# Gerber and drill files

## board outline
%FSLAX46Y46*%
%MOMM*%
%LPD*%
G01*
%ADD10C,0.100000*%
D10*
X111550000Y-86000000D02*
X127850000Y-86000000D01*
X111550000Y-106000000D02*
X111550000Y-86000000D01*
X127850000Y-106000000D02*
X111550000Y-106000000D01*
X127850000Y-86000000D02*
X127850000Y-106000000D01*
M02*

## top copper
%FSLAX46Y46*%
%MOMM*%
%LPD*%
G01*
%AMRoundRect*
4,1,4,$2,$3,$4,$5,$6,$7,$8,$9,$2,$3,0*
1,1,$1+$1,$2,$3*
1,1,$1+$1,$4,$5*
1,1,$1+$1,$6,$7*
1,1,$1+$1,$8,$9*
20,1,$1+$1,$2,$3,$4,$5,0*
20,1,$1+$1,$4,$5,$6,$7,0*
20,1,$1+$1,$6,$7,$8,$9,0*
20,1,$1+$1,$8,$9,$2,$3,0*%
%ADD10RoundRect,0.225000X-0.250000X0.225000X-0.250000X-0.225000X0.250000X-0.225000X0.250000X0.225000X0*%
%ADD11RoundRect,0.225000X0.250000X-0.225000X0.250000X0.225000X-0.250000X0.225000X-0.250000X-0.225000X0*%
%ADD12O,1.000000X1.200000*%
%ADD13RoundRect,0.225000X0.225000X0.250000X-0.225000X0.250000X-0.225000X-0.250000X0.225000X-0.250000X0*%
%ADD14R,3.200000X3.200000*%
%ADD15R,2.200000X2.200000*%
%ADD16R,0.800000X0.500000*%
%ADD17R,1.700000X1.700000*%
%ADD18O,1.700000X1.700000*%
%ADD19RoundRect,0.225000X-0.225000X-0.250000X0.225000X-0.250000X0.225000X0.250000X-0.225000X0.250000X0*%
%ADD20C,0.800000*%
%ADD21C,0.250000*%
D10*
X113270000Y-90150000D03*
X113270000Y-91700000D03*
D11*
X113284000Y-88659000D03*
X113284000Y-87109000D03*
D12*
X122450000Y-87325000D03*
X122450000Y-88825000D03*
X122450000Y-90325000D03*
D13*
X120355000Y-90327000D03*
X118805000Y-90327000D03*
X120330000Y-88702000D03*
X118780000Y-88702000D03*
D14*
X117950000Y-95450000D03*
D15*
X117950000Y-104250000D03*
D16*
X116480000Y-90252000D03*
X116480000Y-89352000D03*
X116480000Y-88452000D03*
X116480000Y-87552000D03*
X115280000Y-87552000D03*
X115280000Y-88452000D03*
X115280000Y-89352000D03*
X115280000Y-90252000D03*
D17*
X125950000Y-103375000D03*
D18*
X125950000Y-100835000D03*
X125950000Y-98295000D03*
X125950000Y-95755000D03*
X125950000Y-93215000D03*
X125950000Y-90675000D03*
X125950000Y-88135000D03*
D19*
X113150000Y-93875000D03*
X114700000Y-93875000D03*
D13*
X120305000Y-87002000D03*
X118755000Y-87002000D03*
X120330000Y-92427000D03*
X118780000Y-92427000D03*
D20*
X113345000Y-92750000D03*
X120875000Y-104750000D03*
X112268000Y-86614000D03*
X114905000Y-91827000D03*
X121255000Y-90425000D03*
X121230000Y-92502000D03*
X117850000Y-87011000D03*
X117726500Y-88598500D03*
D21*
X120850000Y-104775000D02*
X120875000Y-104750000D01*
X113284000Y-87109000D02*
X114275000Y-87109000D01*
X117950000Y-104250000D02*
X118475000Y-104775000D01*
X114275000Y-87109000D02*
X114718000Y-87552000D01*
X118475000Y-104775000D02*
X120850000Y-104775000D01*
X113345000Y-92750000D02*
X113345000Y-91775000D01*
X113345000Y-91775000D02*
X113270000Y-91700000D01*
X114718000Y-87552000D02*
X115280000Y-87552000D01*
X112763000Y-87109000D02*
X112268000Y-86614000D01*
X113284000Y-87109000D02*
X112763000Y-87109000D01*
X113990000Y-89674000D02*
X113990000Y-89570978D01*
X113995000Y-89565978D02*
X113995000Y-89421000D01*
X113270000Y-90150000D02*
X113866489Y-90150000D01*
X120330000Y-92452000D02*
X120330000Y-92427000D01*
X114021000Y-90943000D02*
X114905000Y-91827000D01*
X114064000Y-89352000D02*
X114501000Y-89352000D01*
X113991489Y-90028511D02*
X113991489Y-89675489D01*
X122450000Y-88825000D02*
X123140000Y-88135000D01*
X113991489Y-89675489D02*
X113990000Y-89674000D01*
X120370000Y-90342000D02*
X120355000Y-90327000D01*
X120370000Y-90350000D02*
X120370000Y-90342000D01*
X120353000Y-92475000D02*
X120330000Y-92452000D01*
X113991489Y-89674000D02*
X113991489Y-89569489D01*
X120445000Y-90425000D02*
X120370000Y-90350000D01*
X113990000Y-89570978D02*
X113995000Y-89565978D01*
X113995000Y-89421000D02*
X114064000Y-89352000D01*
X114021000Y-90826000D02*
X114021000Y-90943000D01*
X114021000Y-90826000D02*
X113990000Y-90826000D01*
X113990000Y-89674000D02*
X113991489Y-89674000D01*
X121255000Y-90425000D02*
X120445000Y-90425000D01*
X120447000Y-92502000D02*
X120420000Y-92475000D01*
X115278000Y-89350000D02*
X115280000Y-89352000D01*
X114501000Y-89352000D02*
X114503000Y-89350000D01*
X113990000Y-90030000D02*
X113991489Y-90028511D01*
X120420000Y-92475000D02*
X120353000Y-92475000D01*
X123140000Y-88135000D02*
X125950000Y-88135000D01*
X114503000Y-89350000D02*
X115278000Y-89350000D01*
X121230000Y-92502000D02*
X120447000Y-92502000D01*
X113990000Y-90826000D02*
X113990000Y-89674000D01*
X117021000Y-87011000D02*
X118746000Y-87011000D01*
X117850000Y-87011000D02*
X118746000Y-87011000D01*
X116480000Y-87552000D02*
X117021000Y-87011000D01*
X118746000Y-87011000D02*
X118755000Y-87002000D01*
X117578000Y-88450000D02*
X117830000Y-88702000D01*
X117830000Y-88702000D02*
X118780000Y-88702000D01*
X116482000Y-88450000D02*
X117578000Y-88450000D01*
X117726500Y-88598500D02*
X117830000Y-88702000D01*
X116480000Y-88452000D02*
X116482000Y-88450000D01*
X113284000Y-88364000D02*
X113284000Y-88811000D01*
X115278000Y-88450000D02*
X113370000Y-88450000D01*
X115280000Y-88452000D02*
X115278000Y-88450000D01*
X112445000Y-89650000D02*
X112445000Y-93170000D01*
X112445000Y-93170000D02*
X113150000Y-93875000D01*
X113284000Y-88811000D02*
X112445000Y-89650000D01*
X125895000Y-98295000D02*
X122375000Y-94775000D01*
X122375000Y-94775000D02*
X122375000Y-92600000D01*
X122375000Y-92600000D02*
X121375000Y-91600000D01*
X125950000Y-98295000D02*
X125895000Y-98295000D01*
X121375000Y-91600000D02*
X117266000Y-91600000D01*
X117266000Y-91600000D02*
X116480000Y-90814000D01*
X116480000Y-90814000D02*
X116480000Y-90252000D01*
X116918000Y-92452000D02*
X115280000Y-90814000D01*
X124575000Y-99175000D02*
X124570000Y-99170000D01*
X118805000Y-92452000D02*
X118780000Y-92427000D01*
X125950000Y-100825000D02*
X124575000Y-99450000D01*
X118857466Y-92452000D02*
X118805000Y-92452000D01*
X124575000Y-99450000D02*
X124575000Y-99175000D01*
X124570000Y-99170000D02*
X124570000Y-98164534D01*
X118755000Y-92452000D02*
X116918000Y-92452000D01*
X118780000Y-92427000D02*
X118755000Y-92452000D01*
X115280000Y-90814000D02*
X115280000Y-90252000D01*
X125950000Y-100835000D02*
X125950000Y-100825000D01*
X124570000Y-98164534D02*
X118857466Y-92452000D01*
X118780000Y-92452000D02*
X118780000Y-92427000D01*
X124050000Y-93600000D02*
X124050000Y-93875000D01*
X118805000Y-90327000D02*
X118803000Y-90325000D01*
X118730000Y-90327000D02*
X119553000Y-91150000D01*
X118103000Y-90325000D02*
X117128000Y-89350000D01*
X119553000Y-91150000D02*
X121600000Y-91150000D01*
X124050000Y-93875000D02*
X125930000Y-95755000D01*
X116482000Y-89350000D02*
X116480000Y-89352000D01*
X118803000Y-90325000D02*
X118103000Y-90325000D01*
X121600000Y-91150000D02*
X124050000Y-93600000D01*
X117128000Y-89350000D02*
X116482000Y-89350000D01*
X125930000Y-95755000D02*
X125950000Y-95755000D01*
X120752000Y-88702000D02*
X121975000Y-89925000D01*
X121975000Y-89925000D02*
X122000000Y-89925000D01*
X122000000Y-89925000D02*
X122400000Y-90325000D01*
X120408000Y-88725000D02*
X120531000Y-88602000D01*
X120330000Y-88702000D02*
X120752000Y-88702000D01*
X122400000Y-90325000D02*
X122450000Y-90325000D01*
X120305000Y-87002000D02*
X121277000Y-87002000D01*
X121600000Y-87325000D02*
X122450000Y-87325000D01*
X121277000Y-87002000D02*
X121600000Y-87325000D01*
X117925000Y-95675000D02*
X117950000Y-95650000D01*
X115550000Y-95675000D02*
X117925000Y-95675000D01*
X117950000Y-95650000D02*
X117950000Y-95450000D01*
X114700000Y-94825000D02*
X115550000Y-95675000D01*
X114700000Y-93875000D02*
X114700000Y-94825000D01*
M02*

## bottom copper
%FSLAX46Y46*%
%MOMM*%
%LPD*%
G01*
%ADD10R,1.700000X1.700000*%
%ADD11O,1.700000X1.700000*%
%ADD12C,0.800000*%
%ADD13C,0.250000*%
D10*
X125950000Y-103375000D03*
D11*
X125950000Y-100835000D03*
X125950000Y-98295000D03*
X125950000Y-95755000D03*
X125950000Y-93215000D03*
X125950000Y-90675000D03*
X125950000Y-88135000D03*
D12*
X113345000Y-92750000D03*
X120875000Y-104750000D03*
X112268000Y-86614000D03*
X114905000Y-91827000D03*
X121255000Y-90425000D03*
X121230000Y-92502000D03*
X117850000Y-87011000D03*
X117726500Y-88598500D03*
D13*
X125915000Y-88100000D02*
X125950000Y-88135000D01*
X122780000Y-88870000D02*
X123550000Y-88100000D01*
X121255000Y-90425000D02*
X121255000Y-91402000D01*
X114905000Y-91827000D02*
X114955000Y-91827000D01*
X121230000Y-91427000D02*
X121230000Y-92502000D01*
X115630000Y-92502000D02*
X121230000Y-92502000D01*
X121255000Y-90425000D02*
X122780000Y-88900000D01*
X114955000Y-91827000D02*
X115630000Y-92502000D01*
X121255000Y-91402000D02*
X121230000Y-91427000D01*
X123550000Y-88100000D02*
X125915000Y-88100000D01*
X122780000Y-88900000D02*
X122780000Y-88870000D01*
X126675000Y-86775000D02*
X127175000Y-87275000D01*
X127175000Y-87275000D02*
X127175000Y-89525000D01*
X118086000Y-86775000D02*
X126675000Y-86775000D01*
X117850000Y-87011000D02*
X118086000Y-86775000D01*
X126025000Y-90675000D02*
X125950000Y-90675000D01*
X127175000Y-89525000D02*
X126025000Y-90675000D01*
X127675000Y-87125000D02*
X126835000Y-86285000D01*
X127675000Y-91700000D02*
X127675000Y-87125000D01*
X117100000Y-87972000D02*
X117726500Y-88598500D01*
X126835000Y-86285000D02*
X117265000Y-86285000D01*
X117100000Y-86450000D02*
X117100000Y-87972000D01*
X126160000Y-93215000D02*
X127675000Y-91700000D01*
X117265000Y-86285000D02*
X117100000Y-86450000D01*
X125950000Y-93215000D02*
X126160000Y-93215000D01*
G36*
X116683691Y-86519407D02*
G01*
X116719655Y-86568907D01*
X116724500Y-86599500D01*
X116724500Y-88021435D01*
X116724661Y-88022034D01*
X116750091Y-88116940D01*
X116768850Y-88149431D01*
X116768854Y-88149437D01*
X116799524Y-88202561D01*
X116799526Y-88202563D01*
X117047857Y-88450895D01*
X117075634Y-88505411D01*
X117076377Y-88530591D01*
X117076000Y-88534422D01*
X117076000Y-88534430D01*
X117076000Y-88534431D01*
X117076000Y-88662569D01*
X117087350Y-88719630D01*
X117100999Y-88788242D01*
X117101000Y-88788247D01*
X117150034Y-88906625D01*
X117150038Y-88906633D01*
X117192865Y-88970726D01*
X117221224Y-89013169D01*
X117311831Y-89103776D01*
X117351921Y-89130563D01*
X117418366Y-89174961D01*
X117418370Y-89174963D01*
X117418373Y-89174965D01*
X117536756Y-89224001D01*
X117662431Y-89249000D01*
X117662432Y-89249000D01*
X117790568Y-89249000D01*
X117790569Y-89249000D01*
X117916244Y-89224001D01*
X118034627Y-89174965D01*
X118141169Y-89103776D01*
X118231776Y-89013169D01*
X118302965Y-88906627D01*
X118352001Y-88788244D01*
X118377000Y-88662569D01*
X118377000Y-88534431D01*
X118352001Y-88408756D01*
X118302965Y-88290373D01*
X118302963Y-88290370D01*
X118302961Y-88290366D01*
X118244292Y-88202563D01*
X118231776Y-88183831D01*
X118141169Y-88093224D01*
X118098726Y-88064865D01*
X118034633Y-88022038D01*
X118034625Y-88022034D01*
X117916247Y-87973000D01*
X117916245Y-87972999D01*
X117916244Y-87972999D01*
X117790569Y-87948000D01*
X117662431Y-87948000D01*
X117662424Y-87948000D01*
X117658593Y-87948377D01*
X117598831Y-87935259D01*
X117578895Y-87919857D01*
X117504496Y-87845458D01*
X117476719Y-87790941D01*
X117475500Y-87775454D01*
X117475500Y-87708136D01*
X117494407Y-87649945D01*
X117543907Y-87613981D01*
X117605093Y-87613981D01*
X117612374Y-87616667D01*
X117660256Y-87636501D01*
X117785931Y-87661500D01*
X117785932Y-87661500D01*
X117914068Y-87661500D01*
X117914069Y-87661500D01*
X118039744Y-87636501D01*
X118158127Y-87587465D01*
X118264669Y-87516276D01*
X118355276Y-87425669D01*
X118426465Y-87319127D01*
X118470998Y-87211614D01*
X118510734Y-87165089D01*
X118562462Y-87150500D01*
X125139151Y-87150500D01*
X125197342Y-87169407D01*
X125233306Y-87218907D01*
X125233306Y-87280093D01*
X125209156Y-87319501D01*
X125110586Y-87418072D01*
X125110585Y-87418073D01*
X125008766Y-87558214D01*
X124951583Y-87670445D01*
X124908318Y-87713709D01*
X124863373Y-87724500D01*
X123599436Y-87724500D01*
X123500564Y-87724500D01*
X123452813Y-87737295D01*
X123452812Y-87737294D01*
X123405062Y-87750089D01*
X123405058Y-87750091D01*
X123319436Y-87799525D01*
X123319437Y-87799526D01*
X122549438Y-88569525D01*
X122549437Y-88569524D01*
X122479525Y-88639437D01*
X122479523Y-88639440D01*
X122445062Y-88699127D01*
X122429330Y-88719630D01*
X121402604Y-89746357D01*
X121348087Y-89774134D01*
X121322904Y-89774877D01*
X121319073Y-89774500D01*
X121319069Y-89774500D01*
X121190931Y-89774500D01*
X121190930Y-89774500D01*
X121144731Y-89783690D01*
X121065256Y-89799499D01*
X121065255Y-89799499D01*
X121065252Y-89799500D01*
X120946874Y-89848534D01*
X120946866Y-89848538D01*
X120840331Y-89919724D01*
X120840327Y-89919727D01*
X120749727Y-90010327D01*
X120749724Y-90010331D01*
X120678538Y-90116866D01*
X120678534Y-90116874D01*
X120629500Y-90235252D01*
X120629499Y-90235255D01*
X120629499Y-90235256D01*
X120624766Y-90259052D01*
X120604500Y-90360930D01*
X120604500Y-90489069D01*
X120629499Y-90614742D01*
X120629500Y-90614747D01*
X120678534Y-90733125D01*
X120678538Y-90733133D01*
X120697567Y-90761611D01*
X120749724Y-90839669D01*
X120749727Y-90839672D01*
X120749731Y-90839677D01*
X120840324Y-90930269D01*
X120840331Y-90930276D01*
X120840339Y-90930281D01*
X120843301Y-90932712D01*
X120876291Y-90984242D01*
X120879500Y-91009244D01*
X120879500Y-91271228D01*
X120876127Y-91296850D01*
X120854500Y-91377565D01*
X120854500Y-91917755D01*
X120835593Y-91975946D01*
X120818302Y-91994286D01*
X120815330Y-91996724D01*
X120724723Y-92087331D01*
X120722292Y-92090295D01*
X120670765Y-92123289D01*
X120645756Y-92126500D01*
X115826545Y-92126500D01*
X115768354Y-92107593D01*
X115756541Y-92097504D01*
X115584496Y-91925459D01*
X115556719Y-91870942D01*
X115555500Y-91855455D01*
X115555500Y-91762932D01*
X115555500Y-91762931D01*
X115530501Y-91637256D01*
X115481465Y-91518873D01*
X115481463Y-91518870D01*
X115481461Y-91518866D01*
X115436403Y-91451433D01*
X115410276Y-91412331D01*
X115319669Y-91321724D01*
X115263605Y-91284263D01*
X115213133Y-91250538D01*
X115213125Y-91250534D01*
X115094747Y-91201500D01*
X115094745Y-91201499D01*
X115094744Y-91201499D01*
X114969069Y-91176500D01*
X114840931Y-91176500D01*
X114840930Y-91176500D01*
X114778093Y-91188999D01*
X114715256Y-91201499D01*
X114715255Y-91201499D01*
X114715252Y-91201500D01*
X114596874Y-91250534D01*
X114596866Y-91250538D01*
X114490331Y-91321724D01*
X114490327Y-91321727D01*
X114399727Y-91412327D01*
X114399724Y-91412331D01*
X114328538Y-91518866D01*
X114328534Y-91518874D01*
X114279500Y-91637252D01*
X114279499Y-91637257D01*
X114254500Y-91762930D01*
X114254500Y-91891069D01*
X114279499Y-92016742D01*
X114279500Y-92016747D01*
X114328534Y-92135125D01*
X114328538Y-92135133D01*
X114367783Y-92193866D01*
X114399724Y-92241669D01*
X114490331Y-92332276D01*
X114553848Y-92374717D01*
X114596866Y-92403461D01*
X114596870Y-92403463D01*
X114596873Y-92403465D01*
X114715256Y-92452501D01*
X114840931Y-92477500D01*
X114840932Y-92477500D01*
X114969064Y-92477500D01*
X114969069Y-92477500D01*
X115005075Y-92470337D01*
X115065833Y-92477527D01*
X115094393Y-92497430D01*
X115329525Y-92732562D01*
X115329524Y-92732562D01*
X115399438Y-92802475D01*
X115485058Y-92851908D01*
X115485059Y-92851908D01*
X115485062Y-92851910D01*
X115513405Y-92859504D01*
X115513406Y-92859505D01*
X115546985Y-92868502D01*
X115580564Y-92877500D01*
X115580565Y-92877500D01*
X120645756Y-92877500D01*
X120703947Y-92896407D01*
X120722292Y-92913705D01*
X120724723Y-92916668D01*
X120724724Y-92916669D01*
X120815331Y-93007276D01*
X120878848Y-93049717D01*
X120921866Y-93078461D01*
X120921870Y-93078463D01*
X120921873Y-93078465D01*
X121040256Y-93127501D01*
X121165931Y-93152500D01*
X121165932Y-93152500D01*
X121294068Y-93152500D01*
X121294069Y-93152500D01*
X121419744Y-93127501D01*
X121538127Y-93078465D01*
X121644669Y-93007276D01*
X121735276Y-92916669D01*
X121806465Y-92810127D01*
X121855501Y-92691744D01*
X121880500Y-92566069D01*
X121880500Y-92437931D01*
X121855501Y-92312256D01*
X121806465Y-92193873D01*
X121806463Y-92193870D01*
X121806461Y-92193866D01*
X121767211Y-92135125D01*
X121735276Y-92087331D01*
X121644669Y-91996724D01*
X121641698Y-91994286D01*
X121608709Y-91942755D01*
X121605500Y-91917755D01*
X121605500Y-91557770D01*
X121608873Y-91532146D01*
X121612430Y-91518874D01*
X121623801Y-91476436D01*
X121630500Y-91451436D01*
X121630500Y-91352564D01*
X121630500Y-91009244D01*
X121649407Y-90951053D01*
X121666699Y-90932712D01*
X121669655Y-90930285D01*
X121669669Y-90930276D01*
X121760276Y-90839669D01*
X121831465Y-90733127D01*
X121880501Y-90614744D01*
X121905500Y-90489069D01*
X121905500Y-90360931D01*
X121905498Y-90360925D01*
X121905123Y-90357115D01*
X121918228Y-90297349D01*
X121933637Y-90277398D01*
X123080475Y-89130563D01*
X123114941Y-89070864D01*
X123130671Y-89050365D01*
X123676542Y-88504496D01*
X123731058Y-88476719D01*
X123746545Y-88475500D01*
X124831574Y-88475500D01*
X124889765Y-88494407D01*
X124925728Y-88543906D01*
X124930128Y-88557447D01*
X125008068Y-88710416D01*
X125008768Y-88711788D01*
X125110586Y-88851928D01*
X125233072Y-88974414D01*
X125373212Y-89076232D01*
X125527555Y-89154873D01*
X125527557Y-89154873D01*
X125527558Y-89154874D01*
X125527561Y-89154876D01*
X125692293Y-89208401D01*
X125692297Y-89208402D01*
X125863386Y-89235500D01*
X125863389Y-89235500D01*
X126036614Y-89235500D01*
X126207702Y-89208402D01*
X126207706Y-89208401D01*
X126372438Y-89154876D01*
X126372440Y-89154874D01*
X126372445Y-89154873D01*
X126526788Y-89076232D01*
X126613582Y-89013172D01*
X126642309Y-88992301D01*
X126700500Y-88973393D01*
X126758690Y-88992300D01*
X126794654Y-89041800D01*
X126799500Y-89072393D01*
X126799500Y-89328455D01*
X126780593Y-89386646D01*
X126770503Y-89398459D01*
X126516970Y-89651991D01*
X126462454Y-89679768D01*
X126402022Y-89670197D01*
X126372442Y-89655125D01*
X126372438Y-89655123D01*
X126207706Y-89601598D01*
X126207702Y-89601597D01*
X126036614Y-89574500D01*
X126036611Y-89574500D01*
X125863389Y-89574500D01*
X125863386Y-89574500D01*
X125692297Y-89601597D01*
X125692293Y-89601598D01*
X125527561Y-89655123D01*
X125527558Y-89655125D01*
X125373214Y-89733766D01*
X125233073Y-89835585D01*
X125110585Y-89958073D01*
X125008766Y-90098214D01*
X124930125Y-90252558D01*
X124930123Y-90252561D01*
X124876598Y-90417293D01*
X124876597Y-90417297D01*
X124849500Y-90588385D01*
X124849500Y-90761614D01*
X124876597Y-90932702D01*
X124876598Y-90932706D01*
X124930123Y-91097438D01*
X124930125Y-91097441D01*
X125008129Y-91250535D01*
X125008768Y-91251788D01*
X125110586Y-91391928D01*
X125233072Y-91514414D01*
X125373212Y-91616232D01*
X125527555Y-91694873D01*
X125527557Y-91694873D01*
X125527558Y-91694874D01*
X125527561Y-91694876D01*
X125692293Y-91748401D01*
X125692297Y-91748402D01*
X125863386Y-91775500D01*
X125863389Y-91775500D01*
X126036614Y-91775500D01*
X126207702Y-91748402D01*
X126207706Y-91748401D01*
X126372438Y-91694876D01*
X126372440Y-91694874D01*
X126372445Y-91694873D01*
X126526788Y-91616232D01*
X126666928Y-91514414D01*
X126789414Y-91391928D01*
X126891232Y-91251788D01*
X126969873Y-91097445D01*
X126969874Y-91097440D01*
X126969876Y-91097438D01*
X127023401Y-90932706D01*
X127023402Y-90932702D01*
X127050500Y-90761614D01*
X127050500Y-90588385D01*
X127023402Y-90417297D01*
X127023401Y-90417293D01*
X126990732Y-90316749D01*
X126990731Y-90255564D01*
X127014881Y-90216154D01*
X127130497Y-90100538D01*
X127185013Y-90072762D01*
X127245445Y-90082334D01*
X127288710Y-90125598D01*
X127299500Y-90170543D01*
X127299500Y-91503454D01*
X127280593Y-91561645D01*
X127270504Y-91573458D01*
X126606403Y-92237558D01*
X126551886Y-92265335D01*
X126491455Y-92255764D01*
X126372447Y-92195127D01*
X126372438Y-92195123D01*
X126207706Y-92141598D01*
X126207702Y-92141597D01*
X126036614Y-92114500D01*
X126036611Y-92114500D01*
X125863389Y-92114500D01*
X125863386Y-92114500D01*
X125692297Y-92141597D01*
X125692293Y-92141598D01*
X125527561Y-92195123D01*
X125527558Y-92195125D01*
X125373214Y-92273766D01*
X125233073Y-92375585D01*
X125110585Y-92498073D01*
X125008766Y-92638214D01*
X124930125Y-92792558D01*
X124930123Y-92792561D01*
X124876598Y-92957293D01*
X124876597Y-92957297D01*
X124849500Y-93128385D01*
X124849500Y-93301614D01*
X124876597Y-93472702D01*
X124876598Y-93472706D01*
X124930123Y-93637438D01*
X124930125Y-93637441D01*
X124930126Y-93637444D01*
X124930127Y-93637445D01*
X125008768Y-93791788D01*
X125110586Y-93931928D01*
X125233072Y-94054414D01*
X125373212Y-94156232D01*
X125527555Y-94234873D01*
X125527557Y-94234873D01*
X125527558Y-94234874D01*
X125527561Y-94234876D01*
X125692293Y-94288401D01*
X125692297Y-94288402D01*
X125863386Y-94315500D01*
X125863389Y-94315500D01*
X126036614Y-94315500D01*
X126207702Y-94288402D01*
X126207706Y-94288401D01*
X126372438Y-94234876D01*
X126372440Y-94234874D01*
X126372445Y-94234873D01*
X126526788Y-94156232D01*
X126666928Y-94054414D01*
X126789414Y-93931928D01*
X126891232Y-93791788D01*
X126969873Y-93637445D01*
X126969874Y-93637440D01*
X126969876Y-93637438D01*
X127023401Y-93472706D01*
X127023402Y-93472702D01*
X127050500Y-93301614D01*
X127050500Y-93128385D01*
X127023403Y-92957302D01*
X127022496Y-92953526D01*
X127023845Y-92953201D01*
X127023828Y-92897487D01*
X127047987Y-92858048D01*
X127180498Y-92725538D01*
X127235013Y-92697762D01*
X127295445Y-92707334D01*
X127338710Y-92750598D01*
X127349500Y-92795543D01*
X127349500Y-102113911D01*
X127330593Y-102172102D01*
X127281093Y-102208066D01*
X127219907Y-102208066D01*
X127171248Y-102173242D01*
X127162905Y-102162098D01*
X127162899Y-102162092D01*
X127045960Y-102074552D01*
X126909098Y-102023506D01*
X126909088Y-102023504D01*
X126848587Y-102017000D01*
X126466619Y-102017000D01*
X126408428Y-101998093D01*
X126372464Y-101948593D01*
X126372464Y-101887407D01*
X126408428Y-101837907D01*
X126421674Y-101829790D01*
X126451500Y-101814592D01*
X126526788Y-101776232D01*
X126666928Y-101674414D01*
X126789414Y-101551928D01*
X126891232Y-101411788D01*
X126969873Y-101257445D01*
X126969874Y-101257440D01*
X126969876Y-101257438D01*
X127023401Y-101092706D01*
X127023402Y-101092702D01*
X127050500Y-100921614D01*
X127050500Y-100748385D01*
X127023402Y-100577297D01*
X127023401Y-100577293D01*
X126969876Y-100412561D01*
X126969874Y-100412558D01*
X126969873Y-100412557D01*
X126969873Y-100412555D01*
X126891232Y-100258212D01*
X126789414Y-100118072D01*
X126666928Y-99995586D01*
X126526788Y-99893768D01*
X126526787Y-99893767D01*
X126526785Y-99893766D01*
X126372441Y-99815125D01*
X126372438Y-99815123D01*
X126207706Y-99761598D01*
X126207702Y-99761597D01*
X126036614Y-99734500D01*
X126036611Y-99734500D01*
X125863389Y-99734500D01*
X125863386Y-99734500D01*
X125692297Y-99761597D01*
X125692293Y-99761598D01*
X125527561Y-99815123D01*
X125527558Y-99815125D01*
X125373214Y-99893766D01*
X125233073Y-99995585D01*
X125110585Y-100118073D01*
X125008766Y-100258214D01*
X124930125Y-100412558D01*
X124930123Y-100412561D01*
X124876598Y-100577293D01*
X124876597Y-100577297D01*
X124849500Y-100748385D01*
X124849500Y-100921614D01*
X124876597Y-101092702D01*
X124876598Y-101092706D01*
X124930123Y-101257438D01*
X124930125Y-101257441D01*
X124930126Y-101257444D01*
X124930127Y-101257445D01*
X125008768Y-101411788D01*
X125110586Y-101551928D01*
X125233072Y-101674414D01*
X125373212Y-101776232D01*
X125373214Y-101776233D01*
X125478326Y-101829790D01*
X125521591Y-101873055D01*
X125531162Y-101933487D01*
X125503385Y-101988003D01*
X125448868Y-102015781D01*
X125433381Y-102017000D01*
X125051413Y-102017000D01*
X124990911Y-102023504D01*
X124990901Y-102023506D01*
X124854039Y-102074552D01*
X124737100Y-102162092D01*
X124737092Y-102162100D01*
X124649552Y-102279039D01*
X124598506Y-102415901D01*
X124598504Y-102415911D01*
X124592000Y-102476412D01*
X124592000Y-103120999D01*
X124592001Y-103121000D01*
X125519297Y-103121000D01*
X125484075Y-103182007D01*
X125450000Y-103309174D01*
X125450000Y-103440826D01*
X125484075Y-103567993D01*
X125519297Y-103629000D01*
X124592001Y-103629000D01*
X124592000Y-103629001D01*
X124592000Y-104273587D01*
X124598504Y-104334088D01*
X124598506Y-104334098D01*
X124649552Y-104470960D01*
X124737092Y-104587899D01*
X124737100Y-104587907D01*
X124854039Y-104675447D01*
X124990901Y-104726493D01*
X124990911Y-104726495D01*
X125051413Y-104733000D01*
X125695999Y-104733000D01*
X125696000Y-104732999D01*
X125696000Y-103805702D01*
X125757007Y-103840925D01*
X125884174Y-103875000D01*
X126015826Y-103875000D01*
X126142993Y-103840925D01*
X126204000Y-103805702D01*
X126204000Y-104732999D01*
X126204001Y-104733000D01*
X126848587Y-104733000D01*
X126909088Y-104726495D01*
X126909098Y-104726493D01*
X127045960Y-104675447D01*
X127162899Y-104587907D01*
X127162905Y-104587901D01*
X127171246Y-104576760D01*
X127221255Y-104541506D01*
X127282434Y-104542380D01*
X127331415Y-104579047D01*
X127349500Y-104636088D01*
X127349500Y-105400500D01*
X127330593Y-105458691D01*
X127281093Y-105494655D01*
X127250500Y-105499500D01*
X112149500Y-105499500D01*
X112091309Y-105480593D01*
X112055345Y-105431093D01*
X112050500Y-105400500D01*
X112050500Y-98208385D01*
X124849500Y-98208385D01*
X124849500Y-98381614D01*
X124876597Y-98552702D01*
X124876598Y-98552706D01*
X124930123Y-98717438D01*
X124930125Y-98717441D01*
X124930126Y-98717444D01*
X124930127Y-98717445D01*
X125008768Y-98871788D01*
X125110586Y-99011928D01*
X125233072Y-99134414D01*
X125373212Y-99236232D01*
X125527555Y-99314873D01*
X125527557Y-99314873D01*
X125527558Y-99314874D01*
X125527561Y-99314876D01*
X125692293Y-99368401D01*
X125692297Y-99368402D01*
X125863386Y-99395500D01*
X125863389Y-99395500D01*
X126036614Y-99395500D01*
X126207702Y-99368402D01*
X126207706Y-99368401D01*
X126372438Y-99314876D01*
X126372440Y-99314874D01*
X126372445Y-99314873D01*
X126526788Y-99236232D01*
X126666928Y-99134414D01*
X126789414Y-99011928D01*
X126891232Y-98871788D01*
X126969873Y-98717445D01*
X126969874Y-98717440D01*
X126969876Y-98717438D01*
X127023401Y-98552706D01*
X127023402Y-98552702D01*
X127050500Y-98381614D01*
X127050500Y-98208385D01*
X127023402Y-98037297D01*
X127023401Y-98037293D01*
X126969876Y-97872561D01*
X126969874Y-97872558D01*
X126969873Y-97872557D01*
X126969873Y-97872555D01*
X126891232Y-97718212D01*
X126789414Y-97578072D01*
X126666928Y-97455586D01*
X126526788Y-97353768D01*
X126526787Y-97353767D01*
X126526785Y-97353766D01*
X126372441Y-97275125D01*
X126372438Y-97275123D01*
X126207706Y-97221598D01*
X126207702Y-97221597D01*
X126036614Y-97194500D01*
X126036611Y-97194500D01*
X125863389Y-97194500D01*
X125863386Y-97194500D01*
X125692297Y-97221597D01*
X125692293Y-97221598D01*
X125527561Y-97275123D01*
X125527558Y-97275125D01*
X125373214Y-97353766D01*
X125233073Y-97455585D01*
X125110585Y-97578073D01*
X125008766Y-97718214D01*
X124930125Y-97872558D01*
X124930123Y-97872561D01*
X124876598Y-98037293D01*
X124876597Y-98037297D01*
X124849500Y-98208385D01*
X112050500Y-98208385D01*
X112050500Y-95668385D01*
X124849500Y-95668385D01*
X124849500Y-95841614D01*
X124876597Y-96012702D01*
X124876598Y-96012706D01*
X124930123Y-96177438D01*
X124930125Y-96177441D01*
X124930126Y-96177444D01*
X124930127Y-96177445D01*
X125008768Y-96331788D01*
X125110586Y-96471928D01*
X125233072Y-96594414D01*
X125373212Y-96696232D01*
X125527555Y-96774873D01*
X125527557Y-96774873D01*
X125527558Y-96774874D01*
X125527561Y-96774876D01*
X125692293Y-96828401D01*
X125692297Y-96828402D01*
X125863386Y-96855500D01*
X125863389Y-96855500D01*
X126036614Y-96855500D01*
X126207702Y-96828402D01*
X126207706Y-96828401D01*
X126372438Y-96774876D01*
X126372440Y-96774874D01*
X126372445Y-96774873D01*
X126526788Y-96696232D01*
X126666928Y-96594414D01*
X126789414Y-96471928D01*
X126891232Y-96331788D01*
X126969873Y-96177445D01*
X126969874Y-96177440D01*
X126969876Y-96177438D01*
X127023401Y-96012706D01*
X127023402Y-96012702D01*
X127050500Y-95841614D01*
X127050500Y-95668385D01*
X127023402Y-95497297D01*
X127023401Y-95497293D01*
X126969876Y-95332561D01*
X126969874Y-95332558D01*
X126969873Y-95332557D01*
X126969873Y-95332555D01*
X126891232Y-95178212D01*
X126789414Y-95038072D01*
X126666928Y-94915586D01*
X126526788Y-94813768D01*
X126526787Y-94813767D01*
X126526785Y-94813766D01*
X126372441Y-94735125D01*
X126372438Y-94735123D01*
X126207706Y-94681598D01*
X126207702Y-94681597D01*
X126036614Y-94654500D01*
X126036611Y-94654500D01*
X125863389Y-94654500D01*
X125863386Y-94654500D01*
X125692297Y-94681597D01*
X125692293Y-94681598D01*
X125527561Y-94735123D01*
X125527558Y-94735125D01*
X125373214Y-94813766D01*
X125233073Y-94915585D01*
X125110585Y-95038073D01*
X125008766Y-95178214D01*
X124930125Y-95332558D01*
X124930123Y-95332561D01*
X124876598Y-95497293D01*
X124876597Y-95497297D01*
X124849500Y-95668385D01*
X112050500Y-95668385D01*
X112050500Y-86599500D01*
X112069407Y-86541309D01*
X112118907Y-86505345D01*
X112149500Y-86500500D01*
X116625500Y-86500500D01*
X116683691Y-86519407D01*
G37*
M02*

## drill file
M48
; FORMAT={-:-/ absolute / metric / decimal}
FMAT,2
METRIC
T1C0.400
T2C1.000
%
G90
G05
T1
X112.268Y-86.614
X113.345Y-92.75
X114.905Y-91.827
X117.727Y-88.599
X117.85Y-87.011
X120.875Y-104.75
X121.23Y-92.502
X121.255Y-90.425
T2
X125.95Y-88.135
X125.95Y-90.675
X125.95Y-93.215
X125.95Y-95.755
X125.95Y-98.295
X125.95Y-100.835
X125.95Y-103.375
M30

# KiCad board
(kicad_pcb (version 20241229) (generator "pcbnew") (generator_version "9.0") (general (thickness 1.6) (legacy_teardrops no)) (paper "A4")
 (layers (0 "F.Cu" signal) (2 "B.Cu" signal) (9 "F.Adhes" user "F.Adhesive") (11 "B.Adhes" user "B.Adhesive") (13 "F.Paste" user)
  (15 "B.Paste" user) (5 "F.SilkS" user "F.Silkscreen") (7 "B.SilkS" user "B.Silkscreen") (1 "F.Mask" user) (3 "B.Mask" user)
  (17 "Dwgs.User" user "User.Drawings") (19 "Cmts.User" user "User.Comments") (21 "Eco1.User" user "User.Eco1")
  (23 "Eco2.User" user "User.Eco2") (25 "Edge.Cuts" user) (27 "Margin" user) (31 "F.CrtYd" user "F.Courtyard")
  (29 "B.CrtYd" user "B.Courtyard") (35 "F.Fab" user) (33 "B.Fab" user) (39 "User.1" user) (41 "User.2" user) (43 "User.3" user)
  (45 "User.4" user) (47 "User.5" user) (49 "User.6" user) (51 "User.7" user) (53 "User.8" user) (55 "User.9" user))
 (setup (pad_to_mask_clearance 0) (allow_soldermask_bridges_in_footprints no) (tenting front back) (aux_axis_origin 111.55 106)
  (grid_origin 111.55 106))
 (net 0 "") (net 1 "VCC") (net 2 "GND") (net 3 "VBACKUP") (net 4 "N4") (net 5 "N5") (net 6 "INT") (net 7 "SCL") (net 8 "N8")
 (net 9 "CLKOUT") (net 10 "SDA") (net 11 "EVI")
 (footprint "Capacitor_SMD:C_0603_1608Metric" (layer "F.Cu") (at 113.27 90.925 -90)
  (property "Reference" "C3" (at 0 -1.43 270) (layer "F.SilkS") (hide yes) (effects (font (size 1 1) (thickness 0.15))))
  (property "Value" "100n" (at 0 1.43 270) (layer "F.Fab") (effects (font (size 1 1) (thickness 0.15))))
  (pad "1" smd roundrect (at -0.775 0 270) (size 0.9 0.95) (layers "F.Cu" "F.Mask" "F.Paste") (roundrect_rratio 0.25) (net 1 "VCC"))
  (pad "2" smd roundrect (at 0.775 0 270) (size 0.9 0.95) (layers "F.Cu" "F.Mask" "F.Paste") (roundrect_rratio 0.25) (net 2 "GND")))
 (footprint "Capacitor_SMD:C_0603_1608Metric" (layer "F.Cu") (at 113.284 87.884 90)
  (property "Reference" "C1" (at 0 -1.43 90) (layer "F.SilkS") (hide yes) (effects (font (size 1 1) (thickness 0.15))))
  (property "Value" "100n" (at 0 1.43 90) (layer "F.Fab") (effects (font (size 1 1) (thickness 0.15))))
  (pad "1" smd roundrect (at -0.775 0 90) (size 0.9 0.95) (layers "F.Cu" "F.Mask" "F.Paste") (roundrect_rratio 0.25) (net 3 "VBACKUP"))
  (pad "2" smd roundrect (at 0.775 0 90) (size 0.9 0.95) (layers "F.Cu" "F.Mask" "F.Paste") (roundrect_rratio 0.25) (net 2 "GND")))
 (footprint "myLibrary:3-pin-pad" (layer "F.Cu") (at 122.45 88.825 -90)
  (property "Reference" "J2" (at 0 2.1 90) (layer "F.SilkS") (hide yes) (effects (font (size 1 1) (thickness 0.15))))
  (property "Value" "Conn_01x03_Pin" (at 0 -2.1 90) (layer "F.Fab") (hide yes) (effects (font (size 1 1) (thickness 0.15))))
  (pad "1" smd oval (at -1.5 0 270) (size 1.2 1) (layers "F.Cu" "F.Mask" "F.Paste") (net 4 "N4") (thermal_bridge_angle 45))
  (pad "2" smd oval (at 0 0 270) (size 1.2 1) (layers "F.Cu" "F.Mask" "F.Paste") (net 1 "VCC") (thermal_bridge_angle 45))
  (pad "3" smd oval (at 1.5 0 270) (size 1.2 1) (layers "F.Cu" "F.Mask" "F.Paste") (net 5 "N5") (thermal_bridge_angle 45)))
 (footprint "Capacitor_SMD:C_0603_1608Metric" (layer "F.Cu") (at 119.58 90.327 180)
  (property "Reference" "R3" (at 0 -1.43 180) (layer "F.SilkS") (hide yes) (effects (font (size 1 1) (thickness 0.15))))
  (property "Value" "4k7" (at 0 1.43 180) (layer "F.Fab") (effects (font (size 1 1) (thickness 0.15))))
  (pad "1" smd roundrect (at -0.775 0 180) (size 0.9 0.95) (layers "F.Cu" "F.Mask" "F.Paste") (roundrect_rratio 0.25) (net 1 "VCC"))
  (pad "2" smd roundrect (at 0.775 0 180) (size 0.9 0.95) (layers "F.Cu" "F.Mask" "F.Paste") (roundrect_rratio 0.25) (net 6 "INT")))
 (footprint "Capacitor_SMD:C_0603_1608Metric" (layer "F.Cu") (at 119.555 88.702 180)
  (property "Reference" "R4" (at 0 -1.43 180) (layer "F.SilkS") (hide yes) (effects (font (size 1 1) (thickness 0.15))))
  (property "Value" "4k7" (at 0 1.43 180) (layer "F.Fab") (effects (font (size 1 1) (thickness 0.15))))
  (pad "1" smd roundrect (at -0.775 0 180) (size 0.9 0.95) (layers "F.Cu" "F.Mask" "F.Paste") (roundrect_rratio 0.25) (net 5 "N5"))
  (pad "2" smd roundrect (at 0.775 0 180) (size 0.9 0.95) (layers "F.Cu" "F.Mask" "F.Paste") (roundrect_rratio 0.25) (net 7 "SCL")))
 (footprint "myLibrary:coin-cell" (layer "F.Cu") (at 117.95 99.85 180)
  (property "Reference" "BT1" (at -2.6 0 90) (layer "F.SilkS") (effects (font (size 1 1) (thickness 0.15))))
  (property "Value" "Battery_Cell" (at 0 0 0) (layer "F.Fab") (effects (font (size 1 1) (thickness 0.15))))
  (pad "1" smd rect (at 0 4.4 180) (size 3.2 3.2) (layers "F.Cu" "F.Mask" "F.Paste") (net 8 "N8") (thermal_bridge_angle 45))
  (pad "2" smd rect (at 0 -4.4 180) (size 2.2 2.2) (layers "F.Cu" "F.Mask" "F.Paste") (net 2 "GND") (thermal_bridge_angle 45)))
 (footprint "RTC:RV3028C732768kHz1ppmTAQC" (layer "F.Cu") (at 115.88 88.902 90)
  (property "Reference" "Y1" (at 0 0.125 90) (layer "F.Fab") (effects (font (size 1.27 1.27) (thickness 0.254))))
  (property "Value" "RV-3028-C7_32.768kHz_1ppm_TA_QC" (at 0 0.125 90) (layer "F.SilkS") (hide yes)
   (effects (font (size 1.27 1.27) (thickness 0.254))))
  (pad "1" smd rect (at -1.35 0.6 90) (size 0.5 0.8) (layers "F.Cu" "F.Mask" "F.Paste") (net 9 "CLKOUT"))
  (pad "2" smd rect (at -0.45 0.6 90) (size 0.5 0.8) (layers "F.Cu" "F.Mask" "F.Paste") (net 6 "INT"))
  (pad "3" smd rect (at 0.45 0.6 90) (size 0.5 0.8) (layers "F.Cu" "F.Mask" "F.Paste") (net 7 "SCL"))
  (pad "4" smd rect (at 1.35 0.6 90) (size 0.5 0.8) (layers "F.Cu" "F.Mask" "F.Paste") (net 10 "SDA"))
  (pad "5" smd rect (at 1.35 -0.6 90) (size 0.5 0.8) (layers "F.Cu" "F.Mask" "F.Paste") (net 2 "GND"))
  (pad "6" smd rect (at 0.45 -0.6 90) (size 0.5 0.8) (layers "F.Cu" "F.Mask" "F.Paste") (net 3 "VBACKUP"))
  (pad "7" smd rect (at -0.45 -0.6 90) (size 0.5 0.8) (layers "F.Cu" "F.Mask" "F.Paste") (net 1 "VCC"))
  (pad "8" smd rect (at -1.35 -0.6 90) (size 0.5 0.8) (layers "F.Cu" "F.Mask" "F.Paste") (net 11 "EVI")))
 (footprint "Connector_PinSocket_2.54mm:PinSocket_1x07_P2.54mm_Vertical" (layer "F.Cu") (at 125.95 103.375 180)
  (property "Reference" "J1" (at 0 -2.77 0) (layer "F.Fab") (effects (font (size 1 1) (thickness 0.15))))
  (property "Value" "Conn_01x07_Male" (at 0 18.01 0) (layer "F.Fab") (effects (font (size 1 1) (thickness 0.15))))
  (pad "1" thru_hole rect (at 0 0 180) (size 1.7 1.7) (drill 1) (layers "*.Cu" "*.Mask") (remove_unused_layers no) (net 2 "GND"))
  (pad "2" thru_hole oval (at 0 2.54 180) (size 1.7 1.7) (drill 1) (layers "*.Cu" "*.Mask") (remove_unused_layers no) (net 11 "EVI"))
  (pad "3" thru_hole oval (at 0 5.08 180) (size 1.7 1.7) (drill 1) (layers "*.Cu" "*.Mask") (remove_unused_layers no) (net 9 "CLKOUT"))
  (pad "4" thru_hole oval (at 0 7.62 180) (size 1.7 1.7) (drill 1) (layers "*.Cu" "*.Mask") (remove_unused_layers no) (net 6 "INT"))
  (pad "5" thru_hole oval (at 0 10.16 180) (size 1.7 1.7) (drill 1) (layers "*.Cu" "*.Mask") (remove_unused_layers no) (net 7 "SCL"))
  (pad "6" thru_hole oval (at 0 12.7 180) (size 1.7 1.7) (drill 1) (layers "*.Cu" "*.Mask") (remove_unused_layers no) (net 10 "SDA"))
  (pad "7" thru_hole oval (at 0 15.24 180) (size 1.7 1.7) (drill 1) (layers "*.Cu" "*.Mask") (remove_unused_layers no) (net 1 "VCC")))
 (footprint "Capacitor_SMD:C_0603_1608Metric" (layer "F.Cu") (at 113.925 93.875)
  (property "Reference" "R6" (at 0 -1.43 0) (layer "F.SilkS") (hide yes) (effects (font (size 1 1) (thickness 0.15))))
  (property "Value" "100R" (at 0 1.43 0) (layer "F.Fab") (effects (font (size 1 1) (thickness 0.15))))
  (pad "1" smd roundrect (at -0.775 0) (size 0.9 0.95) (layers "F.Cu" "F.Mask" "F.Paste") (roundrect_rratio 0.25) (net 3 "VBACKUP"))
  (pad "2" smd roundrect (at 0.775 0) (size 0.9 0.95) (layers "F.Cu" "F.Mask" "F.Paste") (roundrect_rratio 0.25) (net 8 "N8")))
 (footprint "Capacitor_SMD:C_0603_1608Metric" (layer "F.Cu") (at 119.53 87.002 180)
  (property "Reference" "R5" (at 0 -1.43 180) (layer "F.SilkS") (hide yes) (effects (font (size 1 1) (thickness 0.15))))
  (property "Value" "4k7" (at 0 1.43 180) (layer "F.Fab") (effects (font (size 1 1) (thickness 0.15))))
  (pad "1" smd roundrect (at -0.775 0 180) (size 0.9 0.95) (layers "F.Cu" "F.Mask" "F.Paste") (roundrect_rratio 0.25) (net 4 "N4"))
  (pad "2" smd roundrect (at 0.775 0 180) (size 0.9 0.95) (layers "F.Cu" "F.Mask" "F.Paste") (roundrect_rratio 0.25) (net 10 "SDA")))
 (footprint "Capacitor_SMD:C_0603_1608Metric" (layer "F.Cu") (at 119.555 92.427 180)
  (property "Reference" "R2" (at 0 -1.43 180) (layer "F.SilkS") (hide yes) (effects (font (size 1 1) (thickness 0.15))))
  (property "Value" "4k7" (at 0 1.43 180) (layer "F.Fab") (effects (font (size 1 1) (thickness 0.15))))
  (pad "1" smd roundrect (at -0.775 0 180) (size 0.9 0.95) (layers "F.Cu" "F.Mask" "F.Paste") (roundrect_rratio 0.25) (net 1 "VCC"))
  (pad "2" smd roundrect (at 0.775 0 180) (size 0.9 0.95) (layers "F.Cu" "F.Mask" "F.Paste") (roundrect_rratio 0.25) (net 11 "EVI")))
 (gr_line (start 111.55 86) (end 127.85 86) (stroke (width 0.1) (type solid)) (layer "Edge.Cuts"))
 (gr_line (start 111.55 106) (end 111.55 86) (stroke (width 0.1) (type solid)) (layer "Edge.Cuts"))
 (gr_line (start 127.85 106) (end 111.55 106) (stroke (width 0.1) (type solid)) (layer "Edge.Cuts"))
 (gr_line (start 127.85 86) (end 127.85 106) (stroke (width 0.1) (type solid)) (layer "Edge.Cuts"))
 (segment (start 120.85 104.775) (end 120.875 104.75) (width 0.25) (layer "F.Cu") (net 2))
 (segment (start 113.284 87.109) (end 114.275 87.109) (width 0.25) (layer "F.Cu") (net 2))
 (segment (start 117.95 104.25) (end 118.475 104.775) (width 0.25) (layer "F.Cu") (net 2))
 (segment (start 114.275 87.109) (end 114.718 87.552) (width 0.25) (layer "F.Cu") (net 2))
 (segment (start 118.475 104.775) (end 120.85 104.775) (width 0.25) (layer "F.Cu") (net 2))
 (segment (start 113.345 92.75) (end 113.345 91.775) (width 0.25) (layer "F.Cu") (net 2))
 (segment (start 113.345 91.775) (end 113.27 91.7) (width 0.25) (layer "F.Cu") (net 2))
 (segment (start 114.718 87.552) (end 115.28 87.552) (width 0.25) (layer "F.Cu") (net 2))
 (segment (start 112.763 87.109) (end 112.268 86.614) (width 0.25) (layer "F.Cu") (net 2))
 (segment (start 113.284 87.109) (end 112.763 87.109) (width 0.25) (layer "F.Cu") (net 2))
 (via (at 113.345 92.75) (size 0.8) (drill 0.4) (layers "F.Cu" "B.Cu") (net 2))
 (via (at 120.875 104.75) (size 0.8) (drill 0.4) (layers "F.Cu" "B.Cu") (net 2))
 (via (at 112.268 86.614) (size 0.8) (drill 0.4) (layers "F.Cu" "B.Cu") (free yes) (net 2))
 (segment (start 113.99 89.674) (end 113.99 89.570978) (width 0.25) (layer "F.Cu") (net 1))
 (segment (start 113.995 89.565978) (end 113.995 89.421) (width 0.25) (layer "F.Cu") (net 1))
 (segment (start 113.27 90.15) (end 113.866489 90.15) (width 0.25) (layer "F.Cu") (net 1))
 (segment (start 120.33 92.452) (end 120.33 92.427) (width 0.25) (layer "F.Cu") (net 1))
 (segment (start 114.021 90.943) (end 114.905 91.827) (width 0.25) (layer "F.Cu") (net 1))
 (segment (start 114.064 89.352) (end 114.501 89.352) (width 0.25) (layer "F.Cu") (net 1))
 (segment (start 113.991489 90.028511) (end 113.991489 89.675489) (width 0.25) (layer "F.Cu") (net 1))
 (segment (start 122.45 88.825) (end 123.14 88.135) (width 0.25) (layer "F.Cu") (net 1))
 (segment (start 113.991489 89.675489) (end 113.99 89.674) (width 0.25) (layer "F.Cu") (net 1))
 (segment (start 120.37 90.342) (end 120.355 90.327) (width 0.25) (layer "F.Cu") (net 1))
 (segment (start 120.37 90.35) (end 120.37 90.342) (width 0.25) (layer "F.Cu") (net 1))
 (segment (start 120.353 92.475) (end 120.33 92.452) (width 0.25) (layer "F.Cu") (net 1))
 (segment (start 113.991489 89.674) (end 113.991489 89.569489) (width 0.25) (layer "F.Cu") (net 1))
 (segment (start 120.445 90.425) (end 120.37 90.35) (width 0.25) (layer "F.Cu") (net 1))
 (segment (start 113.99 89.570978) (end 113.995 89.565978) (width 0.25) (layer "F.Cu") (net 1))
 (segment (start 113.995 89.421) (end 114.064 89.352) (width 0.25) (layer "F.Cu") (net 1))
 (segment (start 114.021 90.826) (end 114.021 90.943) (width 0.25) (layer "F.Cu") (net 1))
 (segment (start 114.021 90.826) (end 113.99 90.826) (width 0.25) (layer "F.Cu") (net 1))
 (segment (start 113.99 89.674) (end 113.991489 89.674) (width 0.25) (layer "F.Cu") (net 1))
 (segment (start 121.255 90.425) (end 120.445 90.425) (width 0.25) (layer "F.Cu") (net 1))
 (segment (start 120.447 92.502) (end 120.42 92.475) (width 0.25) (layer "F.Cu") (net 1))
 (segment (start 115.278 89.35) (end 115.28 89.352) (width 0.25) (layer "F.Cu") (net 1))
 (segment (start 114.501 89.352) (end 114.503 89.35) (width 0.25) (layer "F.Cu") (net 1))
 (segment (start 113.99 90.03) (end 113.991489 90.028511) (width 0.25) (layer "F.Cu") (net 1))
 (segment (start 120.42 92.475) (end 120.353 92.475) (width 0.25) (layer "F.Cu") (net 1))
 (segment (start 123.14 88.135) (end 125.95 88.135) (width 0.25) (layer "F.Cu") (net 1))
 (segment (start 114.503 89.35) (end 115.278 89.35) (width 0.25) (layer "F.Cu") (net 1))
 (segment (start 121.23 92.502) (end 120.447 92.502) (width 0.25) (layer "F.Cu") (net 1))
 (segment (start 113.99 90.826) (end 113.99 89.674) (width 0.25) (layer "F.Cu") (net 1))
 (via (at 114.905 91.827) (size 0.8) (drill 0.4) (layers "F.Cu" "B.Cu") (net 1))
 (via (at 121.255 90.425) (size 0.8) (drill 0.4) (layers "F.Cu" "B.Cu") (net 1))
 (via (at 121.23 92.502) (size 0.8) (drill 0.4) (layers "F.Cu" "B.Cu") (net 1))
 (segment (start 125.915 88.1) (end 125.95 88.135) (width 0.25) (layer "B.Cu") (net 1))
 (segment (start 122.78 88.87) (end 123.55 88.1) (width 0.25) (layer "B.Cu") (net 1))
 (segment (start 121.255 90.425) (end 121.255 91.402) (width 0.25) (layer "B.Cu") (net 1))
 (segment (start 114.905 91.827) (end 114.955 91.827) (width 0.25) (layer "B.Cu") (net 1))
 (segment (start 121.23 91.427) (end 121.23 92.502) (width 0.25) (layer "B.Cu") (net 1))
 (segment (start 115.63 92.502) (end 121.23 92.502) (width 0.25) (layer "B.Cu") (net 1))
 (segment (start 121.255 90.425) (end 122.78 88.9) (width 0.25) (layer "B.Cu") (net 1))
 (segment (start 114.955 91.827) (end 115.63 92.502) (width 0.25) (layer "B.Cu") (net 1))
 (segment (start 121.255 91.402) (end 121.23 91.427) (width 0.25) (layer "B.Cu") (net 1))
 (segment (start 123.55 88.1) (end 125.915 88.1) (width 0.25) (layer "B.Cu") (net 1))
 (segment (start 122.78 88.9) (end 122.78 88.87) (width 0.25) (layer "B.Cu") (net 1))
 (segment (start 117.021 87.011) (end 118.746 87.011) (width 0.25) (layer "F.Cu") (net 10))
 (segment (start 117.85 87.011) (end 118.746 87.011) (width 0.25) (layer "F.Cu") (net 10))
 (segment (start 116.48 87.552) (end 117.021 87.011) (width 0.25) (layer "F.Cu") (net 10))
 (segment (start 118.746 87.011) (end 118.755 87.002) (width 0.25) (layer "F.Cu") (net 10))
 (via (at 117.85 87.011) (size 0.8) (drill 0.4) (layers "F.Cu" "B.Cu") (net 10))
 (segment (start 126.675 86.775) (end 127.175 87.275) (width 0.25) (layer "B.Cu") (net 10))
 (segment (start 127.175 87.275) (end 127.175 89.525) (width 0.25) (layer "B.Cu") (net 10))
 (segment (start 118.086 86.775) (end 126.675 86.775) (width 0.25) (layer "B.Cu") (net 10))
 (segment (start 117.85 87.011) (end 118.086 86.775) (width 0.25) (layer "B.Cu") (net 10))
 (segment (start 126.025 90.675) (end 125.95 90.675) (width 0.25) (layer "B.Cu") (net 10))
 (segment (start 127.175 89.525) (end 126.025 90.675) (width 0.25) (layer "B.Cu") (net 10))
 (segment (start 117.578 88.45) (end 117.83 88.702) (width 0.25) (layer "F.Cu") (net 7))
 (segment (start 117.83 88.702) (end 118.78 88.702) (width 0.25) (layer "F.Cu") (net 7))
 (segment (start 116.482 88.45) (end 117.578 88.45) (width 0.25) (layer "F.Cu") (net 7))
 (segment (start 117.7265 88.5985) (end 117.83 88.702) (width 0.25) (layer "F.Cu") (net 7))
 (segment (start 116.48 88.452) (end 116.482 88.45) (width 0.25) (layer "F.Cu") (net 7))
 (via (at 117.7265 88.5985) (size 0.8) (drill 0.4) (layers "F.Cu" "B.Cu") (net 7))
 (segment (start 127.675 87.125) (end 126.835 86.285) (width 0.25) (layer "B.Cu") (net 7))
 (segment (start 127.675 91.7) (end 127.675 87.125) (width 0.25) (layer "B.Cu") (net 7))
 (segment (start 117.1 87.972) (end 117.7265 88.5985) (width 0.25) (layer "B.Cu") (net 7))
 (segment (start 126.835 86.285) (end 117.265 86.285) (width 0.25) (layer "B.Cu") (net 7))
 (segment (start 117.1 86.45) (end 117.1 87.972) (width 0.25) (layer "B.Cu") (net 7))
 (segment (start 126.16 93.215) (end 127.675 91.7) (width 0.25) (layer "B.Cu") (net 7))
 (segment (start 117.265 86.285) (end 117.1 86.45) (width 0.25) (layer "B.Cu") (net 7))
 (segment (start 125.95 93.215) (end 126.16 93.215) (width 0.25) (layer "B.Cu") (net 7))
 (segment (start 113.284 88.364) (end 113.284 88.811) (width 0.25) (layer "F.Cu") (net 3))
 (segment (start 115.278 88.45) (end 113.37 88.45) (width 0.25) (layer "F.Cu") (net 3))
 (segment (start 115.28 88.452) (end 115.278 88.45) (width 0.25) (layer "F.Cu") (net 3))
 (segment (start 112.445 89.65) (end 112.445 93.17) (width 0.25) (layer "F.Cu") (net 3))
 (segment (start 112.445 93.17) (end 113.15 93.875) (width 0.25) (layer "F.Cu") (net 3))
 (segment (start 113.284 88.811) (end 112.445 89.65) (width 0.25) (layer "F.Cu") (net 3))
 (segment (start 125.895 98.295) (end 122.375 94.775) (width 0.25) (layer "F.Cu") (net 9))
 (segment (start 122.375 94.775) (end 122.375 92.6) (width 0.25) (layer "F.Cu") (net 9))
 (segment (start 122.375 92.6) (end 121.375 91.6) (width 0.25) (layer "F.Cu") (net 9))
 (segment (start 125.95 98.295) (end 125.895 98.295) (width 0.25) (layer "F.Cu") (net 9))
 (segment (start 121.375 91.6) (end 117.266 91.6) (width 0.25) (layer "F.Cu") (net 9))
 (segment (start 117.266 91.6) (end 116.48 90.814) (width 0.25) (layer "F.Cu") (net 9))
 (segment (start 116.48 90.814) (end 116.48 90.252) (width 0.25) (layer "F.Cu") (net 9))
 (segment (start 116.918 92.452) (end 115.28 90.814) (width 0.25) (layer "F.Cu") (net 11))
 (segment (start 124.575 99.175) (end 124.57 99.17) (width 0.25) (layer "F.Cu") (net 11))
 (segment (start 118.805 92.452) (end 118.78 92.427) (width 0.25) (layer "F.Cu") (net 11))
 (segment (start 125.95 100.825) (end 124.575 99.45) (width 0.25) (layer "F.Cu") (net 11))
 (segment (start 118.857466 92.452) (end 118.805 92.452) (width 0.25) (layer "F.Cu") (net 11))
 (segment (start 124.575 99.45) (end 124.575 99.175) (width 0.25) (layer "F.Cu") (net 11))
 (segment (start 124.57 99.17) (end 124.57 98.164534) (width 0.25) (layer "F.Cu") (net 11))
 (segment (start 118.755 92.452) (end 116.918 92.452) (width 0.25) (layer "F.Cu") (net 11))
 (segment (start 118.78 92.427) (end 118.755 92.452) (width 0.25) (layer "F.Cu") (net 11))
 (segment (start 115.28 90.814) (end 115.28 90.252) (width 0.25) (layer "F.Cu") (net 11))
 (segment (start 125.95 100.835) (end 125.95 100.825) (width 0.25) (layer "F.Cu") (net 11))
 (segment (start 124.57 98.164534) (end 118.857466 92.452) (width 0.25) (layer "F.Cu") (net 11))
 (segment (start 118.78 92.452) (end 118.78 92.427) (width 0.25) (layer "F.Cu") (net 11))
 (segment (start 124.05 93.6) (end 124.05 93.875) (width 0.25) (layer "F.Cu") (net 6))
 (segment (start 118.805 90.327) (end 118.803 90.325) (width 0.25) (layer "F.Cu") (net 6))
 (segment (start 118.73 90.327) (end 119.553 91.15) (width 0.25) (layer "F.Cu") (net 6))
 (segment (start 118.103 90.325) (end 117.128 89.35) (width 0.25) (layer "F.Cu") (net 6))
 (segment (start 119.553 91.15) (end 121.6 91.15) (width 0.25) (layer "F.Cu") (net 6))
 (segment (start 124.05 93.875) (end 125.93 95.755) (width 0.25) (layer "F.Cu") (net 6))
 (segment (start 116.482 89.35) (end 116.48 89.352) (width 0.25) (layer "F.Cu") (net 6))
 (segment (start 118.803 90.325) (end 118.103 90.325) (width 0.25) (layer "F.Cu") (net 6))
 (segment (start 121.6 91.15) (end 124.05 93.6) (width 0.25) (layer "F.Cu") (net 6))
 (segment (start 117.128 89.35) (end 116.482 89.35) (width 0.25) (layer "F.Cu") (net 6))
 (segment (start 125.93 95.755) (end 125.95 95.755) (width 0.25) (layer "F.Cu") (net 6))
 (segment (start 120.752 88.702) (end 121.975 89.925) (width 0.25) (layer "F.Cu") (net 5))
 (segment (start 121.975 89.925) (end 122 89.925) (width 0.25) (layer "F.Cu") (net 5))
 (segment (start 122 89.925) (end 122.4 90.325) (width 0.25) (layer "F.Cu") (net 5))
 (segment (start 120.408 88.725) (end 120.531 88.602) (width 0.25) (layer "F.Cu") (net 5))
 (segment (start 120.33 88.702) (end 120.752 88.702) (width 0.25) (layer "F.Cu") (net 5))
 (segment (start 122.4 90.325) (end 122.45 90.325) (width 0.25) (layer "F.Cu") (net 5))
 (segment (start 120.305 87.002) (end 121.277 87.002) (width 0.25) (layer "F.Cu") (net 4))
 (segment (start 121.6 87.325) (end 122.45 87.325) (width 0.25) (layer "F.Cu") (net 4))
 (segment (start 121.277 87.002) (end 121.6 87.325) (width 0.25) (layer "F.Cu") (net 4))
 (segment (start 117.925 95.675) (end 117.95 95.65) (width 0.25) (layer "F.Cu") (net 8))
 (segment (start 115.55 95.675) (end 117.925 95.675) (width 0.25) (layer "F.Cu") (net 8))
 (segment (start 117.95 95.65) (end 117.95 95.45) (width 0.25) (layer "F.Cu") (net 8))
 (segment (start 114.7 94.825) (end 115.55 95.675) (width 0.25) (layer "F.Cu") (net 8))
 (segment (start 114.7 93.875) (end 114.7 94.825) (width 0.25) (layer "F.Cu") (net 8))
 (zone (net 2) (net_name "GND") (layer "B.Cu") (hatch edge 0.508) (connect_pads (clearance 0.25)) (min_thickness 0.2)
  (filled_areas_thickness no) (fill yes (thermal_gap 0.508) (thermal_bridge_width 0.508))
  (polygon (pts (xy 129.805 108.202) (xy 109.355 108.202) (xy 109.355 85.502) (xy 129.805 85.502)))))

